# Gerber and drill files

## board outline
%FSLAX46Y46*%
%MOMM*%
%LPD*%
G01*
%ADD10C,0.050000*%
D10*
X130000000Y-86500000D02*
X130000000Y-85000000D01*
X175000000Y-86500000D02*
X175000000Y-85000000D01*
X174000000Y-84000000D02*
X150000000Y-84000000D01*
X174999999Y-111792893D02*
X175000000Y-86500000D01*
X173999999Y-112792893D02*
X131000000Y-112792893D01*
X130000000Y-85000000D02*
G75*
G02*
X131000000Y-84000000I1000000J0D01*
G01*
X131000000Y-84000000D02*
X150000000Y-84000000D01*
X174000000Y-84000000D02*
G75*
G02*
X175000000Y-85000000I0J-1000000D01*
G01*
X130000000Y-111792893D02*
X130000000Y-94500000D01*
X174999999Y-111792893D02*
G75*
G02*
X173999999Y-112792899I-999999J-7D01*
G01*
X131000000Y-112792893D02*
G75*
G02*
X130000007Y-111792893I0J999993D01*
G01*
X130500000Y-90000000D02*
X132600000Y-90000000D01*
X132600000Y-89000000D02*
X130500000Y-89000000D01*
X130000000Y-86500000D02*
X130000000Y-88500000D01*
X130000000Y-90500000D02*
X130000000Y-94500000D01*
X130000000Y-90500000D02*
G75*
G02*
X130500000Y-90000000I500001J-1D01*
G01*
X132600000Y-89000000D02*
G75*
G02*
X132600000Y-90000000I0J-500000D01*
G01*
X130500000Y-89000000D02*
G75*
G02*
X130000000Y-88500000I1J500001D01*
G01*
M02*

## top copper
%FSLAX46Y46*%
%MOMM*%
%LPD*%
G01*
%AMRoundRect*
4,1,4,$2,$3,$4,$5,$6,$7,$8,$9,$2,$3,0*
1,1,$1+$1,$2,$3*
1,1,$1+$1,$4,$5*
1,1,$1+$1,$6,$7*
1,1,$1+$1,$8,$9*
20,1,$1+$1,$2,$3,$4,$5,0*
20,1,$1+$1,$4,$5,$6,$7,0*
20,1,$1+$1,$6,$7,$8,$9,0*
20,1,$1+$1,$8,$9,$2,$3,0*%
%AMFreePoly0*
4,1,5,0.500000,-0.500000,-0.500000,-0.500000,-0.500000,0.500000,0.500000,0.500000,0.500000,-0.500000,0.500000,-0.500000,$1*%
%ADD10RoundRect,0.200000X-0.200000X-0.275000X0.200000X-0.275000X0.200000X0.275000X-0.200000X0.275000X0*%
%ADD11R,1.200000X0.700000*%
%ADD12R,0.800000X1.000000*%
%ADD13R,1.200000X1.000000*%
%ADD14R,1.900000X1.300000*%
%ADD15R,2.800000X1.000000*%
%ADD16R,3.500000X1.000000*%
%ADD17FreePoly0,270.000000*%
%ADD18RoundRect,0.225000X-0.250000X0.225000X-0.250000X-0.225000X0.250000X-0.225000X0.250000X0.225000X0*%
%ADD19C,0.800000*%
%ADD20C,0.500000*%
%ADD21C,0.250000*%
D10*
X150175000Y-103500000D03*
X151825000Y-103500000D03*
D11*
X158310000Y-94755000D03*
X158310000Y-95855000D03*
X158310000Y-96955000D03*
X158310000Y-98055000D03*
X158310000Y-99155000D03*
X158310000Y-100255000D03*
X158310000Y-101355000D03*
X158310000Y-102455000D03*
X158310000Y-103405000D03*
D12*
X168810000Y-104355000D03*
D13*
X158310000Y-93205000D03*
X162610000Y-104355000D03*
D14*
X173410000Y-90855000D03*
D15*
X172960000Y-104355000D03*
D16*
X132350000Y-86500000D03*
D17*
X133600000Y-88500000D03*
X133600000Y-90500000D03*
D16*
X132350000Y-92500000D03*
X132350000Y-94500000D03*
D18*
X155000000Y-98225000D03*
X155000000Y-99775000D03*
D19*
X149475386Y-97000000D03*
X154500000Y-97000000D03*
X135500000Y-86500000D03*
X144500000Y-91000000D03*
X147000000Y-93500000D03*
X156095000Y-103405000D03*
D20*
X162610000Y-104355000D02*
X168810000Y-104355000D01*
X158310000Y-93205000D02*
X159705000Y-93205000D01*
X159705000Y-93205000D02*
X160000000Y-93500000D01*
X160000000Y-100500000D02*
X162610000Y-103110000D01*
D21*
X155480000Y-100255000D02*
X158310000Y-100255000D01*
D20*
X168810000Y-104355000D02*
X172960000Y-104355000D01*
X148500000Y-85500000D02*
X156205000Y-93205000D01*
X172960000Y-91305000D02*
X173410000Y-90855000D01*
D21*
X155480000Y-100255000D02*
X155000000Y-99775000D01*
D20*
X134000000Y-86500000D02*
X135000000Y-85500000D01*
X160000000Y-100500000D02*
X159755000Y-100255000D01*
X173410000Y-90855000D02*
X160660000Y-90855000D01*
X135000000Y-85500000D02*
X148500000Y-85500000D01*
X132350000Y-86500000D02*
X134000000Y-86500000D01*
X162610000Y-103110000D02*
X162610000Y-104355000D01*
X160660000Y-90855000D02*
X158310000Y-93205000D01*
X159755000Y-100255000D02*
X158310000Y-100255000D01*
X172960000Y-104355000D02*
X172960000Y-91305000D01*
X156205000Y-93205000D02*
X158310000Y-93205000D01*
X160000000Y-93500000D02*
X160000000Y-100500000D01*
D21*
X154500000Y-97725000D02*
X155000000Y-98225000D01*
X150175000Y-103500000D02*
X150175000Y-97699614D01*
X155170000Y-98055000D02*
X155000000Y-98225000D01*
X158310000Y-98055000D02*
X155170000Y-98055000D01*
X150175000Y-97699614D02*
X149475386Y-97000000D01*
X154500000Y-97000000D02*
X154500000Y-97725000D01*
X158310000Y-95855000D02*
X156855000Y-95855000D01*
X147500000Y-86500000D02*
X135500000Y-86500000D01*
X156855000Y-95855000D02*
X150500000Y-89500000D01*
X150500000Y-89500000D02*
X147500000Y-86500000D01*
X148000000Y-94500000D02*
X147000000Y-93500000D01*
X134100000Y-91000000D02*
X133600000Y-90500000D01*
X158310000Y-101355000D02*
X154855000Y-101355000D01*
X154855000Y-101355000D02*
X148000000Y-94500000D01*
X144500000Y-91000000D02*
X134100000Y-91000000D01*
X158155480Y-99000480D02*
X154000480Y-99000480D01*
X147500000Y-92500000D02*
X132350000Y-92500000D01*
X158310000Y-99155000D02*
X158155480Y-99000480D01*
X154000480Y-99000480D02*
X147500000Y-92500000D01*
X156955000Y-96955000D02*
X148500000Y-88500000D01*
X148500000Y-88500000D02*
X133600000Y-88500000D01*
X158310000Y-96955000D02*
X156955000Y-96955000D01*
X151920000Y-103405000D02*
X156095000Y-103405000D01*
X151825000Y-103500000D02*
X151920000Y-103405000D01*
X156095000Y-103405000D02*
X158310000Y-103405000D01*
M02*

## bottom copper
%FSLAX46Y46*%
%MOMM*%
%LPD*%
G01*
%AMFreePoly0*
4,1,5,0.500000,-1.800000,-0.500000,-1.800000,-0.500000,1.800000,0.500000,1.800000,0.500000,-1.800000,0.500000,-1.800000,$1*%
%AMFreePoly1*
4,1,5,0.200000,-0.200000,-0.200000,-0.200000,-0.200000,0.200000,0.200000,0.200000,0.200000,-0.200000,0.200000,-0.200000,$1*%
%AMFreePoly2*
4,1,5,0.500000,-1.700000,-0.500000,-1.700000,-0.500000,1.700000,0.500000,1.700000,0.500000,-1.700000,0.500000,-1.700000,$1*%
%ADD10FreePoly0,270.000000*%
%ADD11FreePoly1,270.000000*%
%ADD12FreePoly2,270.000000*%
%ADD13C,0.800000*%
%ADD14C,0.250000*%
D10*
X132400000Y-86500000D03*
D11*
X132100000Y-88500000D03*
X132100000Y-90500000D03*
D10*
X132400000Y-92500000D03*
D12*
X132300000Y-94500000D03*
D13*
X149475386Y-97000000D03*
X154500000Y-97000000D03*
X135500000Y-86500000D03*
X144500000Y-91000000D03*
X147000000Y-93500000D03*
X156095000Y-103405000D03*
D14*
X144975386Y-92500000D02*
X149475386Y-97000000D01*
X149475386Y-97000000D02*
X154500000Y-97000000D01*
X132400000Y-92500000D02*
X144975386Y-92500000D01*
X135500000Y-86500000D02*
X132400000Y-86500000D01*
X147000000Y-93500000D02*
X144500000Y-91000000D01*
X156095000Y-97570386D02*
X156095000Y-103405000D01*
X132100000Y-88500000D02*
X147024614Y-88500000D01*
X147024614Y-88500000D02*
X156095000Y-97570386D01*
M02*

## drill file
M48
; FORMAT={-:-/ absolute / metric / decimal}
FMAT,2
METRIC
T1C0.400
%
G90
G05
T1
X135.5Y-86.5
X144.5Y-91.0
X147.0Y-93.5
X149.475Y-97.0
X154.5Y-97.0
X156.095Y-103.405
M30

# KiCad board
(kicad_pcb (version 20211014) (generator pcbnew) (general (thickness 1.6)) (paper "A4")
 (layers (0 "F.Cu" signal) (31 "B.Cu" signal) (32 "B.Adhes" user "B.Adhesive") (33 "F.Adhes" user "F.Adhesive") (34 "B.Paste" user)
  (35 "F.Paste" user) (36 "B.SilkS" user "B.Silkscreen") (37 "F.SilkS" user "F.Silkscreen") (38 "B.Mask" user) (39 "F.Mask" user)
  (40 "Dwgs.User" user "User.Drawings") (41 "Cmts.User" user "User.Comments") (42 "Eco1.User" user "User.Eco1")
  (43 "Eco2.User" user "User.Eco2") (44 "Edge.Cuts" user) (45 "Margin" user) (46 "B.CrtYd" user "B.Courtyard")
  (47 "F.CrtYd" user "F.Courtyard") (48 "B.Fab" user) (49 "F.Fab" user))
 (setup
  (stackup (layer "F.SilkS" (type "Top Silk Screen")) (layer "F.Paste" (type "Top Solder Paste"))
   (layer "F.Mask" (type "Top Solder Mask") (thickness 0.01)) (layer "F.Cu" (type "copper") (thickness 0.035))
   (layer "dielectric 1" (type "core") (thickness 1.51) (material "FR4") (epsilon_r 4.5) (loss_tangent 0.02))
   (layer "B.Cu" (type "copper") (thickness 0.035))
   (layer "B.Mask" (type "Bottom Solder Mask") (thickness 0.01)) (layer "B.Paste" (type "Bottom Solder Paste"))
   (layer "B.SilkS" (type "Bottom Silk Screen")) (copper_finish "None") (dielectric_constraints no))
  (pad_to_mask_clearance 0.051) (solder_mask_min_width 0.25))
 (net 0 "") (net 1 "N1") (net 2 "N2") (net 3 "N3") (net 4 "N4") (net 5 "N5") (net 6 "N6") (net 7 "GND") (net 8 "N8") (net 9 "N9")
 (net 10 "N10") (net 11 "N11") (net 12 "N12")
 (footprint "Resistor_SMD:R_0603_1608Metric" (layer "F.Cu") (at 151 103.5)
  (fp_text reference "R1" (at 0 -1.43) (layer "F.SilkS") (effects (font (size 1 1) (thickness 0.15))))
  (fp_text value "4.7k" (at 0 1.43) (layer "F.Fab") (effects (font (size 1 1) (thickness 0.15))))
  (pad "1" smd roundrect locked (at -0.825 0) (size 0.8 0.95) (layers "F.Cu" "F.Paste" "F.Mask") (roundrect_rratio 0.25) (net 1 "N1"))
  (pad "2" smd roundrect locked (at 0.825 0) (size 0.8 0.95) (layers "F.Cu" "F.Paste" "F.Mask") (roundrect_rratio 0.25) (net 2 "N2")))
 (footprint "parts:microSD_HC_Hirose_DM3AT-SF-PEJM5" (layer "F.Cu") (at 166.56 97.535 90)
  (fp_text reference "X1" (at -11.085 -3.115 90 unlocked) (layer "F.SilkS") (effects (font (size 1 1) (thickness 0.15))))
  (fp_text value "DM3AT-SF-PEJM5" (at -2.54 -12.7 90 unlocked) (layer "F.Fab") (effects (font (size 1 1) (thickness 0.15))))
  (pad "1" smd rect (at 2.78 -8.25 90) (size 0.7 1.2) (layers "F.Cu" "F.Paste" "F.Mask") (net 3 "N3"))
  (pad "2" smd rect (at 1.68 -8.25 90) (size 0.7 1.2) (layers "F.Cu" "F.Paste" "F.Mask") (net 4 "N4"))
  (pad "3" smd rect (at 0.58 -8.25 90) (size 0.7 1.2) (layers "F.Cu" "F.Paste" "F.Mask") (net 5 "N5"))
  (pad "4" smd rect (at -0.52 -8.25 90) (size 0.7 1.2) (layers "F.Cu" "F.Paste" "F.Mask") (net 1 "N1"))
  (pad "5" smd rect (at -1.62 -8.25 90) (size 0.7 1.2) (layers "F.Cu" "F.Paste" "F.Mask") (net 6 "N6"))
  (pad "6" smd rect (at -2.72 -8.25 90) (size 0.7 1.2) (layers "F.Cu" "F.Paste" "F.Mask") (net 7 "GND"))
  (pad "7" smd rect (at -3.82 -8.25 90) (size 0.7 1.2) (layers "F.Cu" "F.Paste" "F.Mask") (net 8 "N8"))
  (pad "8" smd rect (at -4.92 -8.25 90) (size 0.7 1.2) (layers "F.Cu" "F.Paste" "F.Mask") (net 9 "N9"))
  (pad "9" smd rect (at -5.87 -8.25 90) (size 0.7 1.2) (layers "F.Cu" "F.Paste" "F.Mask") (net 2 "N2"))
  (pad "10" smd rect (at -6.82 2.25 90) (size 1 0.8) (layers "F.Cu" "F.Paste" "F.Mask") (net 7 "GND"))
  (pad "11" smd rect (at 4.33 -8.25 90) (size 1 1.2) (layers "F.Cu" "F.Paste" "F.Mask") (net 7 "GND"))
  (pad "11" smd rect (at -6.82 -3.95 90) (size 1 1.2) (layers "F.Cu" "F.Paste" "F.Mask") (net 7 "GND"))
  (pad "11" smd rect (at 6.68 6.85 90) (size 1.3 1.9) (layers "F.Cu" "F.Paste" "F.Mask") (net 7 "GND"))
  (pad "11" smd rect (at -6.82 6.4 90) (size 1 2.8) (layers "F.Cu" "F.Paste" "F.Mask") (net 7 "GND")))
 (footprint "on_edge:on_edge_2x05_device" (layer "F.Cu") (at 130 90.5 -90)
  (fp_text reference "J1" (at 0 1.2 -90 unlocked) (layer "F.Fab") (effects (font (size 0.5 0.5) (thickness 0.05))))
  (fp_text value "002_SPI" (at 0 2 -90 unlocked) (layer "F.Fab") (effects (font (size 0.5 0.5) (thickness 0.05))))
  (fp_line (start -0.5 -0.5) (end -0.5 -2.6) (layer "Edge.Cuts") (width 0.05))
  (fp_line (start -1.5 -2.6) (end -1.5 -0.5) (layer "Edge.Cuts") (width 0.05))
  (fp_line (start -4 0) (end -2 0) (layer "Edge.Cuts") (width 0.05))
  (fp_line (start 0 0) (end 4 0) (layer "Edge.Cuts") (width 0.05))
  (fp_arc (start 0 0) (mid -0.353553 -0.146447) (end -0.5 -0.5) (layer "Edge.Cuts") (width 0.05))
  (fp_arc (start -1.5 -2.6) (mid -1 -3.1) (end -0.5 -2.6) (layer "Edge.Cuts") (width 0.05))
  (fp_arc (start -1.5 -0.5) (mid -1.646447 -0.146447) (end -2 0) (layer "Edge.Cuts") (width 0.05))
  (pad "1" smd rect locked (at -4 -2.35 90) (size 1 3.5) (layers "F.Cu" "F.Mask") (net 7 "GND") (zone_connect 0))
  (pad "2" smd custom locked (at -2 -3.6 270) (size 1 1) (layers "F.Cu" "F.Mask") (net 5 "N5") (zone_connect 0)
   (options (clearance outline) (anchor rect)) (primitives))
  (pad "3" smd custom locked (at 0 -3.6 270) (size 1 1) (layers "F.Cu" "F.Mask") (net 8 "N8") (zone_connect 0)
   (options (clearance outline) (anchor rect)) (primitives))
  (pad "4" smd rect locked (at 2 -2.35 90) (size 1 3.5) (layers "F.Cu" "F.Mask") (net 6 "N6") (zone_connect 0))
  (pad "5" smd rect locked (at 4 -2.35 90) (size 1 3.5) (layers "F.Cu" "F.Mask") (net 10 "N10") (zone_connect 0))
  (pad "6" smd custom locked (at -4 -2.4 270) (size 1 3.6) (layers "B.Cu" "B.Mask") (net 4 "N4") (zone_connect 0)
   (options (clearance outline) (anchor rect)) (primitives))
  (pad "7" smd custom locked (at -2 -2.1 270) (size 0.4 0.4) (layers "B.Cu" "B.Mask") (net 2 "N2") (zone_connect 0)
   (options (clearance outline) (anchor rect)) (primitives))
  (pad "8" smd custom locked (at 0 -2.1 270) (size 0.4 0.4) (layers "B.Cu" "B.Mask") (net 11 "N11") (zone_connect 0)
   (options (clearance outline) (anchor rect)) (primitives))
  (pad "9" smd custom locked (at 2 -2.4 270) (size 1 3.6) (layers "B.Cu" "B.Mask") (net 1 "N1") (zone_connect 0)
   (options (clearance outline) (anchor rect)) (primitives))
  (pad "10" smd custom locked (at 4 -2.3 270) (size 1 3.4) (layers "B.Cu" "B.Mask") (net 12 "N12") (zone_connect 0)
   (options (clearance outline) (anchor rect)) (primitives)))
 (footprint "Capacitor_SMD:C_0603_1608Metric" (layer "F.Cu") (at 155 99 -90)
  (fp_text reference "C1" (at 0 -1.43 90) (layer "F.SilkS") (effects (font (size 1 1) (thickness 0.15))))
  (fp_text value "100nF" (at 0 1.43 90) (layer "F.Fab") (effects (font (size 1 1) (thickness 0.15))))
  (pad "1" smd roundrect locked (at -0.775 0 270) (size 0.9 0.95) (layers "F.Cu" "F.Paste" "F.Mask") (roundrect_rratio 0.25) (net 1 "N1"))
  (pad "2" smd roundrect locked (at 0.775 0 270) (size 0.9 0.95) (layers "F.Cu" "F.Paste" "F.Mask") (roundrect_rratio 0.25) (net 7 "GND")))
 (gr_line (start 130 86.5) (end 130 85) (layer "Edge.Cuts") (width 0.05))
 (gr_line (start 175 86.5) (end 175 85) (layer "Edge.Cuts") (width 0.05))
 (gr_line (start 174 84) (end 150 84) (layer "Edge.Cuts") (width 0.05))
 (gr_line (start 174.999999 111.792893) (end 175 86.5) (layer "Edge.Cuts") (width 0.05))
 (gr_line (start 173.999999 112.792893) (end 131 112.792893) (layer "Edge.Cuts") (width 0.05))
 (gr_arc (start 130 85) (mid 130.292881 84.292881) (end 131 84) (layer "Edge.Cuts") (width 0.05))
 (gr_line (start 131 84) (end 150 84) (layer "Edge.Cuts") (width 0.05))
 (gr_arc (start 174 84) (mid 174.707107 84.292893) (end 175 85) (layer "Edge.Cuts") (width 0.05))
 (gr_line (start 130 111.792893) (end 130 94.5) (layer "Edge.Cuts") (width 0.05))
 (gr_arc (start 174.999999 111.792893) (mid 174.707106 112.5) (end 173.999999 112.792893) (layer "Edge.Cuts") (width 0.05))
 (gr_arc (start 131 112.792893) (mid 130.292893 112.5) (end 130 111.792893) (layer "Edge.Cuts") (width 0.05))
 (segment (start 162.61 104.355) (end 168.81 104.355) (width 0.5) (layer "F.Cu") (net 7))
 (segment (start 158.31 93.205) (end 159.705 93.205) (width 0.5) (layer "F.Cu") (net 7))
 (segment (start 159.705 93.205) (end 160 93.5) (width 0.5) (layer "F.Cu") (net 7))
 (segment (start 160 100.5) (end 162.61 103.11) (width 0.5) (layer "F.Cu") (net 7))
 (segment (start 155.48 100.255) (end 158.31 100.255) (width 0.25) (layer "F.Cu") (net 7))
 (segment (start 168.81 104.355) (end 172.96 104.355) (width 0.5) (layer "F.Cu") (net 7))
 (segment (start 148.5 85.5) (end 156.205 93.205) (width 0.5) (layer "F.Cu") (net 7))
 (segment (start 172.96 91.305) (end 173.41 90.855) (width 0.5) (layer "F.Cu") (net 7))
 (segment (start 155.48 100.255) (end 155 99.775) (width 0.25) (layer "F.Cu") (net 7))
 (segment (start 134 86.5) (end 135 85.5) (width 0.5) (layer "F.Cu") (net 7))
 (segment (start 160 100.5) (end 159.755 100.255) (width 0.5) (layer "F.Cu") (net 7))
 (segment (start 173.41 90.855) (end 160.66 90.855) (width 0.5) (layer "F.Cu") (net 7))
 (segment (start 135 85.5) (end 148.5 85.5) (width 0.5) (layer "F.Cu") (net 7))
 (segment (start 132.35 86.5) (end 134 86.5) (width 0.5) (layer "F.Cu") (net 7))
 (segment (start 162.61 103.11) (end 162.61 104.355) (width 0.5) (layer "F.Cu") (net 7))
 (segment (start 160.66 90.855) (end 158.31 93.205) (width 0.5) (layer "F.Cu") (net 7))
 (segment (start 159.755 100.255) (end 158.31 100.255) (width 0.5) (layer "F.Cu") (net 7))
 (segment (start 172.96 104.355) (end 172.96 91.305) (width 0.5) (layer "F.Cu") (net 7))
 (segment (start 156.205 93.205) (end 158.31 93.205) (width 0.5) (layer "F.Cu") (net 7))
 (segment (start 160 93.5) (end 160 100.5) (width 0.5) (layer "F.Cu") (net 7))
 (segment (start 154.5 97.725) (end 155 98.225) (width 0.25) (layer "F.Cu") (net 1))
 (segment (start 150.175 103.5) (end 150.175 97.699614) (width 0.25) (layer "F.Cu") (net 1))
 (segment (start 155.17 98.055) (end 155 98.225) (width 0.25) (layer "F.Cu") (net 1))
 (segment (start 158.31 98.055) (end 155.17 98.055) (width 0.25) (layer "F.Cu") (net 1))
 (segment (start 150.175 97.699614) (end 149.475386 97) (width 0.25) (layer "F.Cu") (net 1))
 (segment (start 154.5 97) (end 154.5 97.725) (width 0.25) (layer "F.Cu") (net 1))
 (via (at 149.475386 97) (size 0.8) (drill 0.4) (layers "F.Cu" "B.Cu") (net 1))
 (via (at 154.5 97) (size 0.8) (drill 0.4) (layers "F.Cu" "B.Cu") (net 1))
 (segment (start 144.975386 92.5) (end 149.475386 97) (width 0.25) (layer "B.Cu") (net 1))
 (segment (start 149.475386 97) (end 154.5 97) (width 0.25) (layer "B.Cu") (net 1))
 (segment (start 132.4 92.5) (end 144.975386 92.5) (width 0.25) (layer "B.Cu") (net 1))
 (segment (start 158.31 95.855) (end 156.855 95.855) (width 0.25) (layer "F.Cu") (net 4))
 (segment (start 147.5 86.5) (end 135.5 86.5) (width 0.25) (layer "F.Cu") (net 4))
 (segment (start 156.855 95.855) (end 150.5 89.5) (width 0.25) (layer "F.Cu") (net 4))
 (segment (start 150.5 89.5) (end 147.5 86.5) (width 0.25) (layer "F.Cu") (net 4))
 (via (at 135.5 86.5) (size 0.8) (drill 0.4) (layers "F.Cu" "B.Cu") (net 4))
 (segment (start 135.5 86.5) (end 132.4 86.5) (width 0.25) (layer "B.Cu") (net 4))
 (segment (start 148 94.5) (end 147 93.5) (width 0.25) (layer "F.Cu") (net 8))
 (segment (start 134.1 91) (end 133.6 90.5) (width 0.25) (layer "F.Cu") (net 8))
 (segment (start 158.31 101.355) (end 154.855 101.355) (width 0.25) (layer "F.Cu") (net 8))
 (segment (start 154.855 101.355) (end 148 94.5) (width 0.25) (layer "F.Cu") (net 8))
 (segment (start 144.5 91) (end 134.1 91) (width 0.25) (layer "F.Cu") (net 8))
 (via (at 144.5 91) (size 0.8) (drill 0.4) (layers "F.Cu" "B.Cu") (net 8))
 (via (at 147 93.5) (size 0.8) (drill 0.4) (layers "F.Cu" "B.Cu") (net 8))
 (segment (start 147 93.5) (end 144.5 91) (width 0.25) (layer "B.Cu") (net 8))
 (segment (start 158.15548 99.00048) (end 154.00048 99.00048) (width 0.25) (layer "F.Cu") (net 6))
 (segment (start 147.5 92.5) (end 132.35 92.5) (width 0.25) (layer "F.Cu") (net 6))
 (segment (start 158.31 99.155) (end 158.15548 99.00048) (width 0.25) (layer "F.Cu") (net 6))
 (segment (start 154.00048 99.00048) (end 147.5 92.5) (width 0.25) (layer "F.Cu") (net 6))
 (segment (start 156.955 96.955) (end 148.5 88.5) (width 0.25) (layer "F.Cu") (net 5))
 (segment (start 148.5 88.5) (end 133.6 88.5) (width 0.25) (layer "F.Cu") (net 5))
 (segment (start 158.31 96.955) (end 156.955 96.955) (width 0.25) (layer "F.Cu") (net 5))
 (segment (start 151.92 103.405) (end 156.095 103.405) (width 0.25) (layer "F.Cu") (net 2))
 (segment (start 151.825 103.5) (end 151.92 103.405) (width 0.25) (layer "F.Cu") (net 2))
 (segment (start 156.095 103.405) (end 158.31 103.405) (width 0.25) (layer "F.Cu") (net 2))
 (via (at 156.095 103.405) (size 0.8) (drill 0.4) (layers "F.Cu" "B.Cu") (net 2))
 (segment (start 156.095 97.570386) (end 156.095 103.405) (width 0.25) (layer "B.Cu") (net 2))
 (segment (start 132.1 88.5) (end 147.024614 88.5) (width 0.25) (layer "B.Cu") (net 2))
 (segment (start 147.024614 88.5) (end 156.095 97.570386) (width 0.25) (layer "B.Cu") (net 2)))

